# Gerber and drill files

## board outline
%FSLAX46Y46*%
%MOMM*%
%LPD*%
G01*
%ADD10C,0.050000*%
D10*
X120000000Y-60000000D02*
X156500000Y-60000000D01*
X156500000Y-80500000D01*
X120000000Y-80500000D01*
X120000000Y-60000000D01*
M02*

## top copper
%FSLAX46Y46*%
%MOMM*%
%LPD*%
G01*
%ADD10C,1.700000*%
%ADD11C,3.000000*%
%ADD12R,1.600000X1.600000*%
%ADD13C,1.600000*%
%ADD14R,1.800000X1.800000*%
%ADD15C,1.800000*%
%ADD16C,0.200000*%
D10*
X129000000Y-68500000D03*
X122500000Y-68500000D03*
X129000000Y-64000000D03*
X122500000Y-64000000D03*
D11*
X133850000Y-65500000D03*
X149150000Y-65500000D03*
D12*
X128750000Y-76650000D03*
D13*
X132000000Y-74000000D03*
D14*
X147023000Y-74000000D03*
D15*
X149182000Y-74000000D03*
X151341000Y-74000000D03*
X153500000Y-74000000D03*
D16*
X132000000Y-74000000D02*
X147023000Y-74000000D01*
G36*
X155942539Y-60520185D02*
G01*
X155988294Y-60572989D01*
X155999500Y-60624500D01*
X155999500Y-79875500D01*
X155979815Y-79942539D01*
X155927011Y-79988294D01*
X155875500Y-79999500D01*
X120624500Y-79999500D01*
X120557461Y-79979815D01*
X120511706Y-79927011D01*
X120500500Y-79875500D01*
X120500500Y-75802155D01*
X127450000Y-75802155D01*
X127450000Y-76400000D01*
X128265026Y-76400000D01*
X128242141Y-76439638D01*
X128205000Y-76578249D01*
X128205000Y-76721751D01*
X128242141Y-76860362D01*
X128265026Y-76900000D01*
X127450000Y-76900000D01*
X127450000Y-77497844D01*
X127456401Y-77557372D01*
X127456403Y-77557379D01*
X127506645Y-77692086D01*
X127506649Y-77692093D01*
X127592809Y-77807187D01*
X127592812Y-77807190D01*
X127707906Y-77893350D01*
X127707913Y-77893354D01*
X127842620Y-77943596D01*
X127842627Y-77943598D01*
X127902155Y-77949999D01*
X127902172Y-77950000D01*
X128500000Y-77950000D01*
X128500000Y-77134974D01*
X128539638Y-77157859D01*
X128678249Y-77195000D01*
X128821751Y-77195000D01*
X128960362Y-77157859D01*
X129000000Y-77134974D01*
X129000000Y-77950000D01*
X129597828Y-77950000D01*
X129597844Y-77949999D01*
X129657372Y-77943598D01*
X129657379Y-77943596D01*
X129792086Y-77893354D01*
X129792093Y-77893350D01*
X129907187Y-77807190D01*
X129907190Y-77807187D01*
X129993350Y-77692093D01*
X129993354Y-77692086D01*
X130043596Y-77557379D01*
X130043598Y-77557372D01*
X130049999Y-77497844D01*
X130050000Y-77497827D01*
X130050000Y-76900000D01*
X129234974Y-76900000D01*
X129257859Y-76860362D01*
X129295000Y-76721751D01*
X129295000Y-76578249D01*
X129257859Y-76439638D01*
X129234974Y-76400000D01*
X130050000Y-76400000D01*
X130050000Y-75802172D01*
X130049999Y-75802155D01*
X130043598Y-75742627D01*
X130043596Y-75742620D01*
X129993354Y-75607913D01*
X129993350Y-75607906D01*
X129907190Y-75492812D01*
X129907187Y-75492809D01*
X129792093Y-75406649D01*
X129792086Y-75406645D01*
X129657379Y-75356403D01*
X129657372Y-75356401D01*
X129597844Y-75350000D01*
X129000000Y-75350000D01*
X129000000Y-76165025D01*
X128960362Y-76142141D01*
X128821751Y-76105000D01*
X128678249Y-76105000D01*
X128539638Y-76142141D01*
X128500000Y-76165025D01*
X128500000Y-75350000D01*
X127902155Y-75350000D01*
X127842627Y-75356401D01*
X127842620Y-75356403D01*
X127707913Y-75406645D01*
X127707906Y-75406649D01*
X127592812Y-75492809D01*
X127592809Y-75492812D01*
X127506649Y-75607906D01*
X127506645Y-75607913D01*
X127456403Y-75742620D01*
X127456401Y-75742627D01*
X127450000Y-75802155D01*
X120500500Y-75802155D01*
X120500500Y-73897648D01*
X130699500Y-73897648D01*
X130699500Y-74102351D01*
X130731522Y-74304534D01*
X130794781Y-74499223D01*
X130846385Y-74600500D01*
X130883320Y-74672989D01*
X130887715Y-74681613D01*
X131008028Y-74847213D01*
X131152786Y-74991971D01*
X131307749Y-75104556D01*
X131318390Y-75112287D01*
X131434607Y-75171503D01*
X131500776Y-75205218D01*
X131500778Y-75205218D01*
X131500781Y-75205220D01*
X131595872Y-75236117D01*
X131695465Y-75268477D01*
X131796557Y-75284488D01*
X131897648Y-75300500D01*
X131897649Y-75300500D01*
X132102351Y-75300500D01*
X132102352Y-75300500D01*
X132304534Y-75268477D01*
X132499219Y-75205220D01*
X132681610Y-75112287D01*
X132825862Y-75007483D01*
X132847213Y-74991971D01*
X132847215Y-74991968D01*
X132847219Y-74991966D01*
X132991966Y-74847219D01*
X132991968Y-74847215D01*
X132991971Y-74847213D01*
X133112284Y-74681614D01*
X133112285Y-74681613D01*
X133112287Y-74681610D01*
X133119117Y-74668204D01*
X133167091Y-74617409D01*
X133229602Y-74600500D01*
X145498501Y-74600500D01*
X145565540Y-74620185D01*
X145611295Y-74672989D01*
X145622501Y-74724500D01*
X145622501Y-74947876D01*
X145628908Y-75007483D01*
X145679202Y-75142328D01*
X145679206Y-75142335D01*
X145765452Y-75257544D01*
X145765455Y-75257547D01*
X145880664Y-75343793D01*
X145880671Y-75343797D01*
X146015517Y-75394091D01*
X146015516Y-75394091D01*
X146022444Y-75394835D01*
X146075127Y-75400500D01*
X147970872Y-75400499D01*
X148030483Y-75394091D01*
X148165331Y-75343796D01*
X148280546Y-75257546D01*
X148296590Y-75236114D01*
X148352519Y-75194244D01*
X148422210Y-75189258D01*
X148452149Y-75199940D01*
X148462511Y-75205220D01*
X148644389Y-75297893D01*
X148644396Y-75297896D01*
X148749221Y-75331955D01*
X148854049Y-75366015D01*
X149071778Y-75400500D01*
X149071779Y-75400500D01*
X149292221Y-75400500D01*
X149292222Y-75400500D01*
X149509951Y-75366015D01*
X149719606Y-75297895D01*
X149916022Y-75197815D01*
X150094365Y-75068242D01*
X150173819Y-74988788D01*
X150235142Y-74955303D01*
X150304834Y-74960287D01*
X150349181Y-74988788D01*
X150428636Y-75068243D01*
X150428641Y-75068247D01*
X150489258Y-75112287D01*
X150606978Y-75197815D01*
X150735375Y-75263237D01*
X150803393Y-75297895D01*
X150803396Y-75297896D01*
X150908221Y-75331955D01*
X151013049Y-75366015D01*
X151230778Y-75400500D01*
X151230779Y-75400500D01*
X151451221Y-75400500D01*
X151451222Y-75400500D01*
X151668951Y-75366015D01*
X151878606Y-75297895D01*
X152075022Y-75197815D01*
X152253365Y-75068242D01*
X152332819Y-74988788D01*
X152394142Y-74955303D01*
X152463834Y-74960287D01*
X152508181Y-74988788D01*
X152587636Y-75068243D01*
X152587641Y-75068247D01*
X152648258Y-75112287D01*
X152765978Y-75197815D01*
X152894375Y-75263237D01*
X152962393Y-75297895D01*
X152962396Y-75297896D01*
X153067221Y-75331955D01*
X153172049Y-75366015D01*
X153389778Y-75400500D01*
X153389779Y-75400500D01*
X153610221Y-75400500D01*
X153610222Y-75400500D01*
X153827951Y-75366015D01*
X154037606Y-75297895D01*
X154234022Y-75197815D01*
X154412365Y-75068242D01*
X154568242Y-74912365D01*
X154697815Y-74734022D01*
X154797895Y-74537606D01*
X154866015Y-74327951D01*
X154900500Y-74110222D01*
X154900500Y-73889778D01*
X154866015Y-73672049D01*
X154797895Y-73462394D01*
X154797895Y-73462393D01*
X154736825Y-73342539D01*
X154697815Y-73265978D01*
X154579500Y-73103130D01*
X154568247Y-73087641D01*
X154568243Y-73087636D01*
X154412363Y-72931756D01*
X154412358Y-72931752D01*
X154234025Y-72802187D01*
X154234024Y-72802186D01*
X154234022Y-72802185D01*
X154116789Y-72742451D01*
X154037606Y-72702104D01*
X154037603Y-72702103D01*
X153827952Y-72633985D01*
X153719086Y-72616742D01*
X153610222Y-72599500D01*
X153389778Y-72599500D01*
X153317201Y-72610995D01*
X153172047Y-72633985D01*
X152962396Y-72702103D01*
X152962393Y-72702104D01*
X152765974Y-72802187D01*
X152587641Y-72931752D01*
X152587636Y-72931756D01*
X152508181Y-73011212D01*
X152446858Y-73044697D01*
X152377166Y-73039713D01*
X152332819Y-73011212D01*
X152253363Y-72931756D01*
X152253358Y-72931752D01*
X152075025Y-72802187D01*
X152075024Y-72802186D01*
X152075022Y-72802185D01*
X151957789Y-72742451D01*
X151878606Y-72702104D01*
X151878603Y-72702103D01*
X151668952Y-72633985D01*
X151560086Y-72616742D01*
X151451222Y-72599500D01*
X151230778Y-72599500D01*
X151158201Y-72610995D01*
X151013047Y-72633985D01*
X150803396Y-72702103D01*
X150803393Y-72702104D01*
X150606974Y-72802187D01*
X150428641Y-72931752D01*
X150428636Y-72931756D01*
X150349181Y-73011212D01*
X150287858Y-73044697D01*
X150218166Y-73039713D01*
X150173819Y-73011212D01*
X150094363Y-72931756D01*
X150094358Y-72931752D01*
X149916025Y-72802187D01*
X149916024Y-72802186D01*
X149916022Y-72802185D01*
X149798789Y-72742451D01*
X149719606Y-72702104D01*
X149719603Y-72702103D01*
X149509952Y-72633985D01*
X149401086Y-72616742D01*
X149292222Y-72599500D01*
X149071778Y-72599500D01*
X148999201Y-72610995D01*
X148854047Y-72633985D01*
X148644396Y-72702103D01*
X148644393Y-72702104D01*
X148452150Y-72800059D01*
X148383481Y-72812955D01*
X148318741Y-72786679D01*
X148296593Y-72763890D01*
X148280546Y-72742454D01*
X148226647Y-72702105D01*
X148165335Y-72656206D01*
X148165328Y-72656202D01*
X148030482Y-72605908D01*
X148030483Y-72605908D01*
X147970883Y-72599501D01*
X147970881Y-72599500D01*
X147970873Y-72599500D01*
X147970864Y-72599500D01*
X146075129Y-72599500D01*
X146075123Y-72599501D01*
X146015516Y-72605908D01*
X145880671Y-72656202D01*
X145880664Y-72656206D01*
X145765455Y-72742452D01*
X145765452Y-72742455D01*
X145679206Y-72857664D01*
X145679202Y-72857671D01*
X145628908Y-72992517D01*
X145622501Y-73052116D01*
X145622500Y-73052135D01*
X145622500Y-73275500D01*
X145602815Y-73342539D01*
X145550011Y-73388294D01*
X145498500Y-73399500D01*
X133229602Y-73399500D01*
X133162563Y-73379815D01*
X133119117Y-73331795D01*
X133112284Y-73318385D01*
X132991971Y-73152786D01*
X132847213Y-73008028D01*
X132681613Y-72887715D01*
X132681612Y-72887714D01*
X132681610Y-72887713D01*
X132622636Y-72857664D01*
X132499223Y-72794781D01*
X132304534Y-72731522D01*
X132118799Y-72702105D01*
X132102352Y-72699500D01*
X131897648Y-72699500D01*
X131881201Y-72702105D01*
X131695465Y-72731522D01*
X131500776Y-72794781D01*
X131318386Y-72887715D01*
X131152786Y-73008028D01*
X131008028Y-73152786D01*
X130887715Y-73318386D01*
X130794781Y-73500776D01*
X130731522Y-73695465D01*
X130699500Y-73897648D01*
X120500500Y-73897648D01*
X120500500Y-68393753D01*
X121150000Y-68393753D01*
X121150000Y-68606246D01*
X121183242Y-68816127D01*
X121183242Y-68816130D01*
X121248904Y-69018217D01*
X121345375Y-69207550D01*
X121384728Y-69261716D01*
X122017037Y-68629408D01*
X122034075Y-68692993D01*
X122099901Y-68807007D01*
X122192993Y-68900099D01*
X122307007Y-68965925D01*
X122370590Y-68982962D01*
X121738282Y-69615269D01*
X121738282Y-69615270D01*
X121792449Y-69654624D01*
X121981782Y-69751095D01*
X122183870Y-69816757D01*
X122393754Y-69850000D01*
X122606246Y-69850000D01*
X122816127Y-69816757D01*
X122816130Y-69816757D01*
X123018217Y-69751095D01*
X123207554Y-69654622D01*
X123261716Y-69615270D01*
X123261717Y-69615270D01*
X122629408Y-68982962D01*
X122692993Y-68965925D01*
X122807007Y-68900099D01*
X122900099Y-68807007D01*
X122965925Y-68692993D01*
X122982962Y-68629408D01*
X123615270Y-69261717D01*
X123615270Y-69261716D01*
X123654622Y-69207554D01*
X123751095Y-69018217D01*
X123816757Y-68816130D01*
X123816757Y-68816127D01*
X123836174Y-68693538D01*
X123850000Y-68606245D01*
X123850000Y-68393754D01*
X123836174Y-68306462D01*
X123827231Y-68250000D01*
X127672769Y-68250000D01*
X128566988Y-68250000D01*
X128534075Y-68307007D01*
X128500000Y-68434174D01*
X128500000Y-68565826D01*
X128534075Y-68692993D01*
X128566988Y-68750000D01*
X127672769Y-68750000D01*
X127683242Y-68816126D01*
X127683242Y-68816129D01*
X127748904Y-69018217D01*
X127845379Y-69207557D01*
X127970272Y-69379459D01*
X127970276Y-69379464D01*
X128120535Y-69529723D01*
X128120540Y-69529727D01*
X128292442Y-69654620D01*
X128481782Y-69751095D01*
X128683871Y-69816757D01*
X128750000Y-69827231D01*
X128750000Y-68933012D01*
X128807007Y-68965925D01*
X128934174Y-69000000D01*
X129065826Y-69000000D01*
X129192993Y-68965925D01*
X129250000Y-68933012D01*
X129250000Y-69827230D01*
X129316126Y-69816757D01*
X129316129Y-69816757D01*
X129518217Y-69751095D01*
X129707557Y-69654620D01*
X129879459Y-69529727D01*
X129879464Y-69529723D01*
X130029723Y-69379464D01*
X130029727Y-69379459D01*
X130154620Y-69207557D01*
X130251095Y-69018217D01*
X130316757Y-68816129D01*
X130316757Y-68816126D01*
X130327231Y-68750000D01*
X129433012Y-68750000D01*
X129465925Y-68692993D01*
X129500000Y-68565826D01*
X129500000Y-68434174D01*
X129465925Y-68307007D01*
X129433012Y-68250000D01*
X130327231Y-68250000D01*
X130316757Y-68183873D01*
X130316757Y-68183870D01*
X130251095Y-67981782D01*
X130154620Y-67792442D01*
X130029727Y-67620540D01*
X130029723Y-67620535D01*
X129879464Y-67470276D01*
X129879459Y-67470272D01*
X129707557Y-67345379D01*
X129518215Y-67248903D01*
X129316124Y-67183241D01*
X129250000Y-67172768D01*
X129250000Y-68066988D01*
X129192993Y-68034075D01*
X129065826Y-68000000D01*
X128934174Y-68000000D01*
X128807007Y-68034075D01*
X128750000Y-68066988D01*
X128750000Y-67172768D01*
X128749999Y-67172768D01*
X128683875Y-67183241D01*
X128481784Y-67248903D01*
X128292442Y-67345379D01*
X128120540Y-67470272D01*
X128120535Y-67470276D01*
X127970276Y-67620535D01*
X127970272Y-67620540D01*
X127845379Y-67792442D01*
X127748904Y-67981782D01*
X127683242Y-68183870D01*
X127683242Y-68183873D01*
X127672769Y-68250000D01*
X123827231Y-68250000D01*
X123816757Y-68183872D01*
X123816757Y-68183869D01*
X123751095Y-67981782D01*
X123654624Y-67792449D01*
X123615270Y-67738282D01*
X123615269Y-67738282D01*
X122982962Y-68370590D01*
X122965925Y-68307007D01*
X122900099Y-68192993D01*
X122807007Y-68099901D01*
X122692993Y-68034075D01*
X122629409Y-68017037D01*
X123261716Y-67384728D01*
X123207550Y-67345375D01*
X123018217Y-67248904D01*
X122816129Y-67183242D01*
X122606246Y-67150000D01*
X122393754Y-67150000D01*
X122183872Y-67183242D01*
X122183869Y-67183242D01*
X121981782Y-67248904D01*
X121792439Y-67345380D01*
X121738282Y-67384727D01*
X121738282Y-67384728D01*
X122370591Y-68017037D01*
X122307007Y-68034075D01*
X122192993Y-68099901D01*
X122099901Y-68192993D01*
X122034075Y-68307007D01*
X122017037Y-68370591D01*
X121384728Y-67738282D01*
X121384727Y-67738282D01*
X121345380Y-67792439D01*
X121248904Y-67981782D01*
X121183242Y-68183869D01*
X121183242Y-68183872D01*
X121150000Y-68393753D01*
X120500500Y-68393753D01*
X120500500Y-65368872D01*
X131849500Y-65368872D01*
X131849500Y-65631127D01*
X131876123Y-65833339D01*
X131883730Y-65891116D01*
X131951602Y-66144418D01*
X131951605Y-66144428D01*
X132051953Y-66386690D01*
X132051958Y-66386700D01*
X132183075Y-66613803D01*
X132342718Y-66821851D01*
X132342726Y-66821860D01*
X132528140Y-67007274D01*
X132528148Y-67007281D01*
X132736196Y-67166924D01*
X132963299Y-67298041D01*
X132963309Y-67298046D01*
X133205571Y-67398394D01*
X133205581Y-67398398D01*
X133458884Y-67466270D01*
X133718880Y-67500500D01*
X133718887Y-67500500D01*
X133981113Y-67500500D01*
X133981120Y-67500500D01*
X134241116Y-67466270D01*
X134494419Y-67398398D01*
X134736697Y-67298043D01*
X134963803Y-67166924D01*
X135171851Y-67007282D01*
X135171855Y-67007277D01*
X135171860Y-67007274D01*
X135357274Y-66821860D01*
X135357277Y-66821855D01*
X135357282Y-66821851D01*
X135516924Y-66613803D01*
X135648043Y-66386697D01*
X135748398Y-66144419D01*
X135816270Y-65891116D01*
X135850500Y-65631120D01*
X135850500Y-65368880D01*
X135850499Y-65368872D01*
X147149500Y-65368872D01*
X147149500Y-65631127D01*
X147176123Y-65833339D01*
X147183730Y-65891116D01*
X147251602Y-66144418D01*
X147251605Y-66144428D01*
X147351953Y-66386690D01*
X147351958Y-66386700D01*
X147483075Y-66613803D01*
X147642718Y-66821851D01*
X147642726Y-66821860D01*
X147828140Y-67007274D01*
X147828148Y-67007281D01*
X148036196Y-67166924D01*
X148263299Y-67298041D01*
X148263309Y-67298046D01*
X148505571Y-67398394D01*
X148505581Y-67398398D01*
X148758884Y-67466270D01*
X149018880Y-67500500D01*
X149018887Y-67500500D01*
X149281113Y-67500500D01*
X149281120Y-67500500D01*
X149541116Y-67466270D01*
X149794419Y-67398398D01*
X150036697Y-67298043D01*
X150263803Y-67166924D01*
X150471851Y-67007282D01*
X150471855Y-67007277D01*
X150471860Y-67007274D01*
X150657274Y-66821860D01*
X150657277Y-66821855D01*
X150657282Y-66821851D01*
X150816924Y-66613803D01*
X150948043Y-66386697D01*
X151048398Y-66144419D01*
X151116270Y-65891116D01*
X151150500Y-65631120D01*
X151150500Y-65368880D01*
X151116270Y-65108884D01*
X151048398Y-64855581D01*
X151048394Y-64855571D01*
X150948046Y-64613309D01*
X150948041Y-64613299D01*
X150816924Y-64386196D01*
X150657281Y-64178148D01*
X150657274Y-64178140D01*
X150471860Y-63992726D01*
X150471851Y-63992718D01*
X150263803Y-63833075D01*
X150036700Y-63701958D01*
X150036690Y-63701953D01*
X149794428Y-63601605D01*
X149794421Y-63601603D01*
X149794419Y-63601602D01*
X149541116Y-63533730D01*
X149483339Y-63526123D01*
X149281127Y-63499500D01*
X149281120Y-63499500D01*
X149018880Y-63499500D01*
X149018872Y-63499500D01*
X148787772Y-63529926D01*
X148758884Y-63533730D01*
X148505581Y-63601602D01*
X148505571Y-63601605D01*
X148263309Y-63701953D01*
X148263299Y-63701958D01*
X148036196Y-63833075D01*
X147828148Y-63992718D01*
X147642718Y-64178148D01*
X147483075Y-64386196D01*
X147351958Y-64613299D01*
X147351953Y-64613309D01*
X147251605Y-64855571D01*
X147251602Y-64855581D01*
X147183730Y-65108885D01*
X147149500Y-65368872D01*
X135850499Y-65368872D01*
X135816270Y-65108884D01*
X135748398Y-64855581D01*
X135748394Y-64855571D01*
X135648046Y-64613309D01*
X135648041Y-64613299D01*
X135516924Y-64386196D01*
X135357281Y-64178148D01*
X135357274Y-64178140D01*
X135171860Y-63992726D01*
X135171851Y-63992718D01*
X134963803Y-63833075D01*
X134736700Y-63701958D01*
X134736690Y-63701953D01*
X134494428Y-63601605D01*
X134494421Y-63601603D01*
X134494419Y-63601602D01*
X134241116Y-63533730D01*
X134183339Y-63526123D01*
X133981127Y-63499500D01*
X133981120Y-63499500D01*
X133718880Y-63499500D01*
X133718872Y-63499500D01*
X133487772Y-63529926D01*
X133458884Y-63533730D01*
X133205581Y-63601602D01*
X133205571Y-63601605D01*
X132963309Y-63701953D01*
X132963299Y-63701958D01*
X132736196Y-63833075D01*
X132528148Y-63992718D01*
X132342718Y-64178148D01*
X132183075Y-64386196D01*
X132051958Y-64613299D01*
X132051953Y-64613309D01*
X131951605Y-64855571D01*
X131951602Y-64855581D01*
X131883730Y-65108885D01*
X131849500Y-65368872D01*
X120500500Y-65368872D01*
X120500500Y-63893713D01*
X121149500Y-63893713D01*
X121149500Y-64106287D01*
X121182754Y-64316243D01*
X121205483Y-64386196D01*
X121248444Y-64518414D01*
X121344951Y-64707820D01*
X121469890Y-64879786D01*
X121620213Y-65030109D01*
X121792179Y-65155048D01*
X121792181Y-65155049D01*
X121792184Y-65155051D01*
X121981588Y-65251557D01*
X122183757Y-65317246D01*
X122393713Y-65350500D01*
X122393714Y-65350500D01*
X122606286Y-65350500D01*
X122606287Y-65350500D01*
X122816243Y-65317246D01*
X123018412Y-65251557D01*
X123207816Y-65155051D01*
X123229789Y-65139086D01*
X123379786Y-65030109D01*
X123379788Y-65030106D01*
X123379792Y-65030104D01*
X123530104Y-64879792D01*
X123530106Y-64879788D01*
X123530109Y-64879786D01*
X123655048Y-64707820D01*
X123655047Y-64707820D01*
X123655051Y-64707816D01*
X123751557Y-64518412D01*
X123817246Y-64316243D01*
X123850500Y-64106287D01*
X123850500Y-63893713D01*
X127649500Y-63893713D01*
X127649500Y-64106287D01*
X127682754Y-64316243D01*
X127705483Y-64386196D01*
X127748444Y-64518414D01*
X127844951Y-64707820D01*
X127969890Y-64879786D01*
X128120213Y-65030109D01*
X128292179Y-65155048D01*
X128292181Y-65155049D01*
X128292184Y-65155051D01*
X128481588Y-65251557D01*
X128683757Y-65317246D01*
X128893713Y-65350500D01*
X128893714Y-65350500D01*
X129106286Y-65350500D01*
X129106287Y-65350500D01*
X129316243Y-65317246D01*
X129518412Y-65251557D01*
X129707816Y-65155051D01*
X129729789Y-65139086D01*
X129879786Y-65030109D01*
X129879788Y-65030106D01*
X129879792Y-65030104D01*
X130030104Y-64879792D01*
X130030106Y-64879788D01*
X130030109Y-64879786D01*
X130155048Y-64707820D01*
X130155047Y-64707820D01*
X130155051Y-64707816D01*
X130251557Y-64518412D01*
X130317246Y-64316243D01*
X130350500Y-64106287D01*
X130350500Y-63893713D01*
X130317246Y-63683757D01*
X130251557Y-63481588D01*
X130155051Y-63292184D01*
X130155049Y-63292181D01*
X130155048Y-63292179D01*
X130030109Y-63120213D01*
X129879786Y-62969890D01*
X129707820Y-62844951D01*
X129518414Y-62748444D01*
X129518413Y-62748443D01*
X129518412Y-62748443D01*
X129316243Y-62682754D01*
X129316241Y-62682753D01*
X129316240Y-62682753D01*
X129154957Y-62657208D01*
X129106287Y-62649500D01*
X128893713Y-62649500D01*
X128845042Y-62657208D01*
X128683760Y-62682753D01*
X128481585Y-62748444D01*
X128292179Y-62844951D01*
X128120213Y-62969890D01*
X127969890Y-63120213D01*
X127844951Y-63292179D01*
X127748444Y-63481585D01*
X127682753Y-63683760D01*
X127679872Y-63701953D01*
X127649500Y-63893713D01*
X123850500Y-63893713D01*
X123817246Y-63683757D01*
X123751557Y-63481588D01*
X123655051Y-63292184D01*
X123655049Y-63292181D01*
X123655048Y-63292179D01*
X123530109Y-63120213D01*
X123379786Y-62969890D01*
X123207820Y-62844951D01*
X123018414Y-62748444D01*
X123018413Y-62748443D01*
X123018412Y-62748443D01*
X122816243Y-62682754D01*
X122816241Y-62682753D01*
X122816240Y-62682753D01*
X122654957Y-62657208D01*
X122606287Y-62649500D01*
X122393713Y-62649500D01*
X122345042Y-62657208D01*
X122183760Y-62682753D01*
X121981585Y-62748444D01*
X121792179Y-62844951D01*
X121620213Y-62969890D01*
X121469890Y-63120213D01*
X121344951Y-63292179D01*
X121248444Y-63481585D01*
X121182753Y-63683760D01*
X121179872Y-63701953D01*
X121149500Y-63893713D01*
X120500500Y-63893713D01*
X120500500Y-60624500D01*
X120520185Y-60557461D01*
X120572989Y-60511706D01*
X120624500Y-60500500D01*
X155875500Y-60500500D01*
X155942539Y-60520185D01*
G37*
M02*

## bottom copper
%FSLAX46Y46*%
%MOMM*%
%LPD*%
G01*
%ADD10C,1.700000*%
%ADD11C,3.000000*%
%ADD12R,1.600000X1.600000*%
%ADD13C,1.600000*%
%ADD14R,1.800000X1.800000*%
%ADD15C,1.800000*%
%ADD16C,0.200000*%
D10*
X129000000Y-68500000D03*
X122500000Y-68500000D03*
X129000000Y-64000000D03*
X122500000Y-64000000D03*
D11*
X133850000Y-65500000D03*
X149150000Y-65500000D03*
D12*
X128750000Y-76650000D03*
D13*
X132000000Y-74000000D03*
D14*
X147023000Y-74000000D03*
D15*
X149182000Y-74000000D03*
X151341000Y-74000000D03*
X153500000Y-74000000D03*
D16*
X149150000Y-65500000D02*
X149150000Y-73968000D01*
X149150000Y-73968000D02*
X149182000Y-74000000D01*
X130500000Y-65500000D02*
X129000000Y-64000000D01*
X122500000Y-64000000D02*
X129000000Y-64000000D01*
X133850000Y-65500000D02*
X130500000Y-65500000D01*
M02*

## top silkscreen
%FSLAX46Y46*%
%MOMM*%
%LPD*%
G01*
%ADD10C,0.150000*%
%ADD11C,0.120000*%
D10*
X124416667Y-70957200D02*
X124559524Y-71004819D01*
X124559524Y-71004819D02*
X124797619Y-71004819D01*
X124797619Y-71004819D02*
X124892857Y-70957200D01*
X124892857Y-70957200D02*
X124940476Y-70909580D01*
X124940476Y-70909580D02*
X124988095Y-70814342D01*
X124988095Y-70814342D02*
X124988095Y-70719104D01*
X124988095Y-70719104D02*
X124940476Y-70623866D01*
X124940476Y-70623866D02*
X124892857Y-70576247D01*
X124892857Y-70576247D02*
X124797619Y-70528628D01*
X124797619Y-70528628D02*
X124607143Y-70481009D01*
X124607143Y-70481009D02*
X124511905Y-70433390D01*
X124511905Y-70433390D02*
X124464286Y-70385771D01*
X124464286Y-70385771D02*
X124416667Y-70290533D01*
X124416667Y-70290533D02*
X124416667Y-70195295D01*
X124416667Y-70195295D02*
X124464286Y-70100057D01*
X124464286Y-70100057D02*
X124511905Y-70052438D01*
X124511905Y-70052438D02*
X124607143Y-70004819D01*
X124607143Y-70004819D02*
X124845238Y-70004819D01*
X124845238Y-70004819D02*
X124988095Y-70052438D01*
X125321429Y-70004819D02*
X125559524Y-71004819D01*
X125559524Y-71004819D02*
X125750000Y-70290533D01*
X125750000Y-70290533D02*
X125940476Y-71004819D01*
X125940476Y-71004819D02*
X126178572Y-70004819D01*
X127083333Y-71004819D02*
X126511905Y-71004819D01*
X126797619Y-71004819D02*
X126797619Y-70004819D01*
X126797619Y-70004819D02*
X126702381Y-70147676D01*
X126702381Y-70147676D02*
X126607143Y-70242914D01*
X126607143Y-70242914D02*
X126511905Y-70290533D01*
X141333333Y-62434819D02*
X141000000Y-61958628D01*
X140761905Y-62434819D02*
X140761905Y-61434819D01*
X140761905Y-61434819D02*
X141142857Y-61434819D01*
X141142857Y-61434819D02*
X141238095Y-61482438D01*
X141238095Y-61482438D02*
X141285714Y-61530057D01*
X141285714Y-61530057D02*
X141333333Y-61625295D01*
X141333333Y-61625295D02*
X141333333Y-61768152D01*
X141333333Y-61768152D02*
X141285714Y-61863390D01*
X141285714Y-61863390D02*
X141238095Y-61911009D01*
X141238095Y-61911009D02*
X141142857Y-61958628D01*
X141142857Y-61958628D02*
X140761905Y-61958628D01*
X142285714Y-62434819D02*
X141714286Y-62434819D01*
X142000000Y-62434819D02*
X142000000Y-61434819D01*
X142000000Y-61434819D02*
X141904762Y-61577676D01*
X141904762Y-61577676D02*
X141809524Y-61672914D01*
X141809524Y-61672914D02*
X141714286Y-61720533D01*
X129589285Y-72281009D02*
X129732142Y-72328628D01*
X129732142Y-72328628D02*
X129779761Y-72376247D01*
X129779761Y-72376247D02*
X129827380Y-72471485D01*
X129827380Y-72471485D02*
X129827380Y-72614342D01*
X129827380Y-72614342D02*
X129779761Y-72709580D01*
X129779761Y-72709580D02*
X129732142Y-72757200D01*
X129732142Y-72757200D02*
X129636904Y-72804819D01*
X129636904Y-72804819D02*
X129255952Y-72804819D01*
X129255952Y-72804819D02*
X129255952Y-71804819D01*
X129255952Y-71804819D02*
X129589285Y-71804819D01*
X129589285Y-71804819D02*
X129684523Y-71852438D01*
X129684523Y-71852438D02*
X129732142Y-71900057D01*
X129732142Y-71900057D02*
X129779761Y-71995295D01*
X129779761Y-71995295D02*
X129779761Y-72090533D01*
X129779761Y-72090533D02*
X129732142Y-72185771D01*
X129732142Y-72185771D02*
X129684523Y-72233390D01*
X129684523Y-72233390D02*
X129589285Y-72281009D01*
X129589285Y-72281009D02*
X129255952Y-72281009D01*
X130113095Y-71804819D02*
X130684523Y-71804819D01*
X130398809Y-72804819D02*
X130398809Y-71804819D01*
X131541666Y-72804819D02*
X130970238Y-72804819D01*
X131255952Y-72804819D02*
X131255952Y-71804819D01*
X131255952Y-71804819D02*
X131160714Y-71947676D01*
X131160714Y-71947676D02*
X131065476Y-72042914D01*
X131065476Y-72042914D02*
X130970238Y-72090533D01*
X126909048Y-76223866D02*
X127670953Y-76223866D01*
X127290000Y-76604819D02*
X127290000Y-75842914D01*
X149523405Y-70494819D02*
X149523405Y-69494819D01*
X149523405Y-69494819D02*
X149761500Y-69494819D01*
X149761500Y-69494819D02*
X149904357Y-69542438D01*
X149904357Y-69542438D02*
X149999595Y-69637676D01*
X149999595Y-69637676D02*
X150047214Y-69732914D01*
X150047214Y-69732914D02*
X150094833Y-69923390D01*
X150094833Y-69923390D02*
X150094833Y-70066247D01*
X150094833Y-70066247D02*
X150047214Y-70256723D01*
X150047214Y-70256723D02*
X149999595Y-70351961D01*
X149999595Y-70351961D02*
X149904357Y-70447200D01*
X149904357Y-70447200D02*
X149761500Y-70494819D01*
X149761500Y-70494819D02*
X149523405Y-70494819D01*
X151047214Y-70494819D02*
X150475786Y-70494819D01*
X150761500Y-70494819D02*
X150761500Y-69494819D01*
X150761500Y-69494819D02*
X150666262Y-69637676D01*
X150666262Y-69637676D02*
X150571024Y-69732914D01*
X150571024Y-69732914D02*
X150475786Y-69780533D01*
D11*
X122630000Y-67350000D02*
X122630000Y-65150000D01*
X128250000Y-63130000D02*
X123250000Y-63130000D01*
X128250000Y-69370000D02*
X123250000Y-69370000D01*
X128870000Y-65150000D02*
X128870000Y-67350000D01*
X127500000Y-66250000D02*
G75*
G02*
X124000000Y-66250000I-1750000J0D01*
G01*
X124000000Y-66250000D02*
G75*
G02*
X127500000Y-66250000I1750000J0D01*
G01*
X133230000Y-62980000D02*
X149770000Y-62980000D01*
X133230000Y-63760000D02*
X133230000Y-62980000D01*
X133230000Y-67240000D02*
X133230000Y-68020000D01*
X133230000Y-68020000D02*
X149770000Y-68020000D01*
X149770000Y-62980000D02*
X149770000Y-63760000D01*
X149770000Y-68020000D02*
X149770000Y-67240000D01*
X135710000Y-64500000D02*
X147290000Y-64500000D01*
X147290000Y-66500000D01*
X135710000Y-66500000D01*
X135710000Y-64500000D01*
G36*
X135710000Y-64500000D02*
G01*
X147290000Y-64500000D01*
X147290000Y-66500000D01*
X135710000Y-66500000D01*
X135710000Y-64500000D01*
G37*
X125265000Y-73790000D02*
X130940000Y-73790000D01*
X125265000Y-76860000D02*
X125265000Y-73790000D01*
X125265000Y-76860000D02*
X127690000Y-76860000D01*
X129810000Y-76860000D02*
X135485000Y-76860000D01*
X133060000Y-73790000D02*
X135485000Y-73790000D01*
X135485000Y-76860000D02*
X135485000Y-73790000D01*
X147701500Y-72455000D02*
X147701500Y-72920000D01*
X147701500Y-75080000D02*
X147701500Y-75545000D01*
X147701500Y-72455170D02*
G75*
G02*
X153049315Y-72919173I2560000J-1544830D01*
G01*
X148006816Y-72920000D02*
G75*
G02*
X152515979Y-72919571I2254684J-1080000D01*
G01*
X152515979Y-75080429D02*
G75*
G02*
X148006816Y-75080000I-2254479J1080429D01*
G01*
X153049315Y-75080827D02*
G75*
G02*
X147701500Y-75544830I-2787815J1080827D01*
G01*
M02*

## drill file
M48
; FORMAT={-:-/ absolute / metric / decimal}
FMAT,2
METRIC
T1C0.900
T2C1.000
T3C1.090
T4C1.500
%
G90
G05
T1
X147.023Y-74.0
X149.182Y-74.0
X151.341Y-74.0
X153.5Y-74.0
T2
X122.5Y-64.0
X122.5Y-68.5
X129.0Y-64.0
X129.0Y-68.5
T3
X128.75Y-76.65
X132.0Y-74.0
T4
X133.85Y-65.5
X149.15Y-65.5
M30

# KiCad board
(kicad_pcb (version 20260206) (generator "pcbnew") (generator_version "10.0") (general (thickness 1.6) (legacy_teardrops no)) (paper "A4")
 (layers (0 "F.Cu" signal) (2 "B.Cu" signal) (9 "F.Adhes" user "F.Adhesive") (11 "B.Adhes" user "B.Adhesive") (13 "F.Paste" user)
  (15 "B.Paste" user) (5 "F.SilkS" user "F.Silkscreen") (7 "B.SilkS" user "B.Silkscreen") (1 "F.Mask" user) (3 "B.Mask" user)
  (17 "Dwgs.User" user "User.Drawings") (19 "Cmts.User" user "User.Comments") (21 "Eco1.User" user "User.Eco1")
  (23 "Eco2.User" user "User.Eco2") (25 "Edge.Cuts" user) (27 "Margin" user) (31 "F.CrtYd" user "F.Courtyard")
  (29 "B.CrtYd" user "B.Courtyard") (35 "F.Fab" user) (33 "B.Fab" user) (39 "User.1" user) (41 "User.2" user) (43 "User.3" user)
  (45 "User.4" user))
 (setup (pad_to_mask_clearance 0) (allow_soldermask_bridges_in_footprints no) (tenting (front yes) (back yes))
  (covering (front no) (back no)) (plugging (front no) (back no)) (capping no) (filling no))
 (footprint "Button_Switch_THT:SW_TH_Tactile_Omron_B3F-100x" (layer "F.Cu") (at 129 68.5 180)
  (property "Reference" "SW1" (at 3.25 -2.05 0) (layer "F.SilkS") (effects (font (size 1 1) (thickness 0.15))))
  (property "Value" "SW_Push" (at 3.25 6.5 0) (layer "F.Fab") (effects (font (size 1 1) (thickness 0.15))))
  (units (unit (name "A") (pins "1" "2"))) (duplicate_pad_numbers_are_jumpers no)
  (fp_line (start 6.37 1.15) (end 6.37 3.35) (stroke (width 0.12) (type solid)) (layer "F.SilkS"))
  (fp_line (start 0.75 5.37) (end 5.75 5.37) (stroke (width 0.12) (type solid)) (layer "F.SilkS"))
  (fp_line (start 0.75 -0.87) (end 5.75 -0.87) (stroke (width 0.12) (type solid)) (layer "F.SilkS"))
  (fp_line (start 0.13 3.35) (end 0.13 1.15) (stroke (width 0.12) (type solid)) (layer "F.SilkS"))
  (fp_circle (center 3.25 2.25) (end 5 2.25) (stroke (width 0.12) (type solid)) (fill no) (layer "F.SilkS"))
  (pad "1" thru_hole circle (at 0 0 180) (size 1.7 1.7) (drill 1) (layers "*.Cu" "*.Mask") (remove_unused_layers no) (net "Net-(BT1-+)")
   (thermal_bridge_angle 90))
  (pad "1" thru_hole circle (at 6.5 0 180) (size 1.7 1.7) (drill 1) (layers "*.Cu" "*.Mask") (remove_unused_layers no) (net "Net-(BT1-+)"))
  (pad "2" thru_hole circle (at 0 4.5 180) (size 1.7 1.7) (drill 1) (layers "*.Cu" "*.Mask") (remove_unused_layers no) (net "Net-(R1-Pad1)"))
  (pad "2" thru_hole circle (at 6.5 4.5 180) (size 1.7 1.7) (drill 1) (layers "*.Cu" "*.Mask") (remove_unused_layers no)
   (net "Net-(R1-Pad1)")))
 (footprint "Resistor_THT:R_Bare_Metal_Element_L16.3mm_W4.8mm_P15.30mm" (layer "F.Cu") (at 133.85 65.5)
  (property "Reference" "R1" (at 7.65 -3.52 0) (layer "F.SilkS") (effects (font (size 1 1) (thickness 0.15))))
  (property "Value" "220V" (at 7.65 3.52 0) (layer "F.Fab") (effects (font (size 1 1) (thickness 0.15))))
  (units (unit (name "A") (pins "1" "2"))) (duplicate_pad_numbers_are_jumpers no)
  (fp_line (start -0.62 -2.52) (end 15.92 -2.52) (stroke (width 0.12) (type solid)) (layer "F.SilkS"))
  (fp_line (start -0.62 -1.74) (end -0.62 -2.52) (stroke (width 0.12) (type solid)) (layer "F.SilkS"))
  (fp_line (start -0.62 1.74) (end -0.62 2.52) (stroke (width 0.12) (type solid)) (layer "F.SilkS"))
  (fp_line (start -0.62 2.52) (end 15.92 2.52) (stroke (width 0.12) (type solid)) (layer "F.SilkS"))
  (fp_line (start 15.92 -2.52) (end 15.92 -1.74) (stroke (width 0.12) (type solid)) (layer "F.SilkS"))
  (fp_line (start 15.92 2.52) (end 15.92 1.74) (stroke (width 0.12) (type solid)) (layer "F.SilkS"))
  (fp_rect (start 1.86 -1) (end 13.44 1) (stroke (width 0.12) (type solid)) (fill yes) (layer "F.SilkS"))
  (pad "1" thru_hole circle (at 0 0) (size 3 3) (drill 1.5) (layers "*.Cu" "*.Mask") (remove_unused_layers no) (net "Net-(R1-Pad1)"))
  (pad "2" thru_hole circle (at 15.3 0) (size 3 3) (drill 1.5) (layers "*.Cu" "*.Mask") (remove_unused_layers no) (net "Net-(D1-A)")))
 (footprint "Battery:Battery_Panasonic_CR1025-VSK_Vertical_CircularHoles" (layer "F.Cu") (at 128.75 76.65)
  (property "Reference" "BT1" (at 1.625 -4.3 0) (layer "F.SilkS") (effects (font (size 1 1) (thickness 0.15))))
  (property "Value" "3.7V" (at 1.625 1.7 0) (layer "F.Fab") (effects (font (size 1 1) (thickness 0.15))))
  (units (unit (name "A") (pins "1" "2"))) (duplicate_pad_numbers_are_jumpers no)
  (fp_line (start -3.485 -2.86) (end 2.19 -2.86) (stroke (width 0.12) (type solid)) (layer "F.SilkS"))
  (fp_line (start -3.485 0.21) (end -3.485 -2.86) (stroke (width 0.12) (type solid)) (layer "F.SilkS"))
  (fp_line (start -3.485 0.21) (end -1.06 0.21) (stroke (width 0.12) (type solid)) (layer "F.SilkS"))
  (fp_line (start 1.06 0.21) (end 6.735 0.21) (stroke (width 0.12) (type solid)) (layer "F.SilkS"))
  (fp_line (start 4.31 -2.86) (end 6.735 -2.86) (stroke (width 0.12) (type solid)) (layer "F.SilkS"))
  (fp_line (start 6.735 0.21) (end 6.735 -2.86) (stroke (width 0.12) (type solid)) (layer "F.SilkS"))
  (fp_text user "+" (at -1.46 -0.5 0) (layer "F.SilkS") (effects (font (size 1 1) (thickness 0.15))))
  (pad "1" thru_hole rect (at 0 0) (size 1.6 1.6) (drill 1.09) (layers "*.Cu" "*.Mask") (remove_unused_layers no) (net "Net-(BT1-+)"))
  (pad "2" thru_hole circle (at 3.25 -2.65) (size 1.6 1.6) (drill 1.09) (layers "*.Cu" "*.Mask") (remove_unused_layers no)
   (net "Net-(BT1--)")))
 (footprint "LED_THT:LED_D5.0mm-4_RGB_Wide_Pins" (layer "F.Cu") (at 147.023 74)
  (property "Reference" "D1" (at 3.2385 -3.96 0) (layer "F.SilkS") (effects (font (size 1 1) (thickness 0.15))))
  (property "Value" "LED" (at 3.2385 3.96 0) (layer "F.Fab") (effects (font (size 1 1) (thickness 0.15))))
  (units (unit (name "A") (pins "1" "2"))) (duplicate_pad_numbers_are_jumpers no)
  (fp_line (start 0.6785 -1.545) (end 0.6785 -1.08) (stroke (width 0.12) (type solid)) (layer "F.SilkS"))
  (fp_line (start 0.6785 1.08) (end 0.6785 1.545) (stroke (width 0.12) (type solid)) (layer "F.SilkS"))
  (fp_arc (start 0.6785 -1.54483) (mid 3.496956 -2.978809) (end 6.026315 -1.080827) (stroke (width 0.12) (type solid)) (layer "F.SilkS"))
  (fp_arc (start 0.983816 -1.08) (mid 3.238262 -2.5) (end 5.492979 -1.080429) (stroke (width 0.12) (type solid)) (layer "F.SilkS"))
  (fp_arc (start 5.492979 1.080429) (mid 3.238262 2.5) (end 0.983816 1.08) (stroke (width 0.12) (type solid)) (layer "F.SilkS"))
  (fp_arc (start 6.026315 1.080827) (mid 3.496956 2.978808) (end 0.6785 1.54483) (stroke (width 0.12) (type solid)) (layer "F.SilkS"))
  (pad "1" thru_hole rect (at 0 0) (size 1.8 1.8) (drill 0.9) (layers "*.Cu" "*.Mask") (remove_unused_layers no) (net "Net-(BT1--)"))
  (pad "2" thru_hole circle (at 2.159 0) (size 1.8 1.8) (drill 0.9) (layers "*.Cu" "*.Mask") (remove_unused_layers no) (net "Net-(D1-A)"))
  (pad "3" thru_hole circle (at 4.318 0) (size 1.8 1.8) (drill 0.9) (layers "*.Cu" "*.Mask") (remove_unused_layers no))
  (pad "4" thru_hole circle (at 6.477 0) (size 1.8 1.8) (drill 0.9) (layers "*.Cu" "*.Mask") (remove_unused_layers no)))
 (gr_rect (start 120 60) (end 156.5 80.5) (stroke (width 0.05) (type default)) (fill no) (layer "Edge.Cuts"))
 (segment (start 132 74) (end 147.023 74) (width 0.2) (layer "F.Cu") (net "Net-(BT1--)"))
 (segment (start 149.15 65.5) (end 149.15 73.968) (width 0.2) (layer "B.Cu") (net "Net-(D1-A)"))
 (segment (start 149.15 73.968) (end 149.182 74) (width 0.2) (layer "B.Cu") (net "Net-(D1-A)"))
 (segment (start 130.5 65.5) (end 129 64) (width 0.2) (layer "B.Cu") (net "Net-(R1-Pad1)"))
 (segment (start 122.5 64) (end 129 64) (width 0.2) (layer "B.Cu") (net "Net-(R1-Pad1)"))
 (segment (start 133.85 65.5) (end 130.5 65.5) (width 0.2) (layer "B.Cu") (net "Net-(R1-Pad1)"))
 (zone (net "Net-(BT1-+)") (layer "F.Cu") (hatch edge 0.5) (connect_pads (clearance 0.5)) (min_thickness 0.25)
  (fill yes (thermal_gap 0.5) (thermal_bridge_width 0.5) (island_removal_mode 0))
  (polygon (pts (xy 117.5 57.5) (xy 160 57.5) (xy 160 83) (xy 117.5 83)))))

